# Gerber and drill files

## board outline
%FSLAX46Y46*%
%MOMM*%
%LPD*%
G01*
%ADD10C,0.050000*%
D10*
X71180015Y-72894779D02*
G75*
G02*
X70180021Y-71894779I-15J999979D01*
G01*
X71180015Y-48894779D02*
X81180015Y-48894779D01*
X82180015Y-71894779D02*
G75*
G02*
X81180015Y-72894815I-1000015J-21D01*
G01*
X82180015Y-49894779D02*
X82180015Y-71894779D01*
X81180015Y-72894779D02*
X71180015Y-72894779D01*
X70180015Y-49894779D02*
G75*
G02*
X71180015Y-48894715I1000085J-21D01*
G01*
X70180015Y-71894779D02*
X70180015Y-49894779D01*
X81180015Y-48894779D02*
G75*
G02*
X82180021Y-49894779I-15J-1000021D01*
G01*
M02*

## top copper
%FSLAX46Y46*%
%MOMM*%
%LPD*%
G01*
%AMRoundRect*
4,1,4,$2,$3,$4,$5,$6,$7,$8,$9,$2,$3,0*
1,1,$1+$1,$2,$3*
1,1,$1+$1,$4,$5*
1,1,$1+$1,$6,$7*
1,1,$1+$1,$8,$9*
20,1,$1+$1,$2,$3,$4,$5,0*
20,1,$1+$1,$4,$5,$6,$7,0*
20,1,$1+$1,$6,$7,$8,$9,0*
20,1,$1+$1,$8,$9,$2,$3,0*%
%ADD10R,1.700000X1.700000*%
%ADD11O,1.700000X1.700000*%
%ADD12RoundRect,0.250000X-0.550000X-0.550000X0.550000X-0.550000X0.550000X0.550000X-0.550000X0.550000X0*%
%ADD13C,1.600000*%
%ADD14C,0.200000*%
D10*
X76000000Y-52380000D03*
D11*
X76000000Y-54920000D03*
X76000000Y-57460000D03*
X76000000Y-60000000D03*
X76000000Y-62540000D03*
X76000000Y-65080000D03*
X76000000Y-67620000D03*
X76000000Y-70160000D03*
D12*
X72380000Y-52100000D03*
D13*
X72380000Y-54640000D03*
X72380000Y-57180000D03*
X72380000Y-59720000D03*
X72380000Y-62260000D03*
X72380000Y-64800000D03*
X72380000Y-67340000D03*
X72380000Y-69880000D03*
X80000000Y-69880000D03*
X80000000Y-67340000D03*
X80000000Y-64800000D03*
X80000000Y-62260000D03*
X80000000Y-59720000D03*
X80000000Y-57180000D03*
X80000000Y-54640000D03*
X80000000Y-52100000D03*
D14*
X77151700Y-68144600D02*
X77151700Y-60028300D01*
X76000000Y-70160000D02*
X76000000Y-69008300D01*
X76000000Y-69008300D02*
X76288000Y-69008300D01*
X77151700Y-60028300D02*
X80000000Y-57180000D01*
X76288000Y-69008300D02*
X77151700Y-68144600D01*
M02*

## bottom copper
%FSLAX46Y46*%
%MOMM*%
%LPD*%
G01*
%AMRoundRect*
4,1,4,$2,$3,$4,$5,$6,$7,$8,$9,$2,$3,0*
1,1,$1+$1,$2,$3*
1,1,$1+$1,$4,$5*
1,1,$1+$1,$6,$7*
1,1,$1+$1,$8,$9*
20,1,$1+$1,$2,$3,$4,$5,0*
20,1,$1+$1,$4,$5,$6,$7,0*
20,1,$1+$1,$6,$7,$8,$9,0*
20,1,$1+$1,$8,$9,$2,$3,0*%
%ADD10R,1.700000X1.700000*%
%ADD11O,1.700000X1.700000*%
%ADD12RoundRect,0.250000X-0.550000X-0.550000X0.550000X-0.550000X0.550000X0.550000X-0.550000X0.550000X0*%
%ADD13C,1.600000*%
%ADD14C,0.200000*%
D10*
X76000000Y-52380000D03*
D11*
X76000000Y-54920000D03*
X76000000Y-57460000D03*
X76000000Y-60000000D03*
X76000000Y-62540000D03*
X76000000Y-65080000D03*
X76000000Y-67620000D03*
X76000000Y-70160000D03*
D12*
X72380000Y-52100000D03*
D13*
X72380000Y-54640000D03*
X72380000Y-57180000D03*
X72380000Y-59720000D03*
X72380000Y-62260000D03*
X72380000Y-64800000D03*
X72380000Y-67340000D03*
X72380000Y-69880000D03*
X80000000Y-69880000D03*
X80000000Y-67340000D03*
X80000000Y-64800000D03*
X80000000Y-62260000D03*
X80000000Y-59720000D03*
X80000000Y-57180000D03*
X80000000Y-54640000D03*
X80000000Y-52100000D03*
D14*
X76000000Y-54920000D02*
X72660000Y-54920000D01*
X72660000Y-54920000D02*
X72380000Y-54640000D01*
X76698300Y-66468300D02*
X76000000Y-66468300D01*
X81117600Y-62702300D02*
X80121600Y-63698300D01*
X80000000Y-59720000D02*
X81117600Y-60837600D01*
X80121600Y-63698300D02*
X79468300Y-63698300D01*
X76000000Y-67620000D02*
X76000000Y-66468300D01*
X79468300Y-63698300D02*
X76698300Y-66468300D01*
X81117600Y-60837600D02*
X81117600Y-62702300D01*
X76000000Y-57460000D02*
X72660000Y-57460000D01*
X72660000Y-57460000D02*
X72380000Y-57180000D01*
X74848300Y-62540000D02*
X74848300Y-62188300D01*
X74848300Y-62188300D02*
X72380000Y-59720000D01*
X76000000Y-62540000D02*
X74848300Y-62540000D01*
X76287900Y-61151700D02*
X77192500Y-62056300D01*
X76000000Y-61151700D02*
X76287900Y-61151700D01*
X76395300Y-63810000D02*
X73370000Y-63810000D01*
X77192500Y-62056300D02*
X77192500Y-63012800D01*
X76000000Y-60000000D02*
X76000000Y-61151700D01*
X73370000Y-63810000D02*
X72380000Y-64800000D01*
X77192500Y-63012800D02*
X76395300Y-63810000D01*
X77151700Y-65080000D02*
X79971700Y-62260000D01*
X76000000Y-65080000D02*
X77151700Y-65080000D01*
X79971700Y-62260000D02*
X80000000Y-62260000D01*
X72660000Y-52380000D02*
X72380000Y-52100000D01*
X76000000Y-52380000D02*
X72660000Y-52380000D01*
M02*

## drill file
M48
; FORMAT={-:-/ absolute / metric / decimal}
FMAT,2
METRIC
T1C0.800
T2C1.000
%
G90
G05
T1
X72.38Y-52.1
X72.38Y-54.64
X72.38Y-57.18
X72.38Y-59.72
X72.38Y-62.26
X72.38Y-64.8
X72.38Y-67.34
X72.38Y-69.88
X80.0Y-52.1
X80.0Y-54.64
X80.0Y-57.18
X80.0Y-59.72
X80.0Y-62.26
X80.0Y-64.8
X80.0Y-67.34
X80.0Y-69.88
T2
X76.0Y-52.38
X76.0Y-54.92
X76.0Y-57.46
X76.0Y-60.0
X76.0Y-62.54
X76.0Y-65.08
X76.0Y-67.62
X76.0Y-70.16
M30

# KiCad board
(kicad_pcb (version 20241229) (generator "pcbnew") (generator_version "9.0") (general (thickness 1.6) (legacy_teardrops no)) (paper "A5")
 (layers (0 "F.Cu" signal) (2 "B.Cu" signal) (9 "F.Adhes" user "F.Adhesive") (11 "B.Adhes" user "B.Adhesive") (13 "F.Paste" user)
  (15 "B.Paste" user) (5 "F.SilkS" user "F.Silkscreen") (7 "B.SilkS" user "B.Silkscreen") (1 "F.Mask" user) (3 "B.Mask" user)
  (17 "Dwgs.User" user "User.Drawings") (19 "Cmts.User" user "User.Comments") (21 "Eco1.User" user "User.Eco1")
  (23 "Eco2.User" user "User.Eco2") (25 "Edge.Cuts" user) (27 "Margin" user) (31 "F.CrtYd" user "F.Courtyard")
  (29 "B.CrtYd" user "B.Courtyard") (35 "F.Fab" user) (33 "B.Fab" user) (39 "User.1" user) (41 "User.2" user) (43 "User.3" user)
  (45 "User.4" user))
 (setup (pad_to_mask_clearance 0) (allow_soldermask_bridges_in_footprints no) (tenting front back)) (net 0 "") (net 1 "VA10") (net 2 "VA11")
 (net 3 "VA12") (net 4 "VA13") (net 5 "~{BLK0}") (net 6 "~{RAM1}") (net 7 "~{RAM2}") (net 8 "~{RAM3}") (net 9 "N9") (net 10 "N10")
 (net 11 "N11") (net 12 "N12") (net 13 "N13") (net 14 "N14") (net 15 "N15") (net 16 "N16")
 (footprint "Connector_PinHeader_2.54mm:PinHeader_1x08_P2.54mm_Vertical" (layer "F.Cu") (at 76 52.38)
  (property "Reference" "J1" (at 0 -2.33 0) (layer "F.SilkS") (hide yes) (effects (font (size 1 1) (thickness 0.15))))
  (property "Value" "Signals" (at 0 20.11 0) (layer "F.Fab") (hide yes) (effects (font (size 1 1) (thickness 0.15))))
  (pad "1" thru_hole rect (at 0 0) (size 1.7 1.7) (drill 1) (layers "*.Cu" "*.Mask") (remove_unused_layers no) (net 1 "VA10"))
  (pad "2" thru_hole oval (at 0 2.54) (size 1.7 1.7) (drill 1) (layers "*.Cu" "*.Mask") (remove_unused_layers no) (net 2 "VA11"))
  (pad "3" thru_hole oval (at 0 5.08) (size 1.7 1.7) (drill 1) (layers "*.Cu" "*.Mask") (remove_unused_layers no) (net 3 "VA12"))
  (pad "4" thru_hole oval (at 0 7.62) (size 1.7 1.7) (drill 1) (layers "*.Cu" "*.Mask") (remove_unused_layers no) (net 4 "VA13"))
  (pad "5" thru_hole oval (at 0 10.16) (size 1.7 1.7) (drill 1) (layers "*.Cu" "*.Mask") (remove_unused_layers no) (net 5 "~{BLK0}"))
  (pad "6" thru_hole oval (at 0 12.7) (size 1.7 1.7) (drill 1) (layers "*.Cu" "*.Mask") (remove_unused_layers no) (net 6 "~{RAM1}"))
  (pad "7" thru_hole oval (at 0 15.24) (size 1.7 1.7) (drill 1) (layers "*.Cu" "*.Mask") (remove_unused_layers no) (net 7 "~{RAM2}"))
  (pad "8" thru_hole oval (at 0 17.78) (size 1.7 1.7) (drill 1) (layers "*.Cu" "*.Mask") (remove_unused_layers no) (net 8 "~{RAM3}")))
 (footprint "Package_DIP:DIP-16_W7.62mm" (layer "F.Cu") (at 72.38 52.1)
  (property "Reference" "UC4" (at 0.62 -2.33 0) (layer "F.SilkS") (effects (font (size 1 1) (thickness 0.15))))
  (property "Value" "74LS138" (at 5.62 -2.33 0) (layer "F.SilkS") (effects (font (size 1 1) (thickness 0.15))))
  (pad "1" thru_hole roundrect (at 0 0) (size 1.6 1.6) (drill 0.8) (layers "*.Cu" "*.Mask") (remove_unused_layers no)
   (roundrect_rratio 0.15625) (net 1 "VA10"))
  (pad "2" thru_hole circle (at 0 2.54) (size 1.6 1.6) (drill 0.8) (layers "*.Cu" "*.Mask") (remove_unused_layers no) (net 2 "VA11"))
  (pad "3" thru_hole circle (at 0 5.08) (size 1.6 1.6) (drill 0.8) (layers "*.Cu" "*.Mask") (remove_unused_layers no) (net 3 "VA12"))
  (pad "4" thru_hole circle (at 0 7.62) (size 1.6 1.6) (drill 0.8) (layers "*.Cu" "*.Mask") (remove_unused_layers no) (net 5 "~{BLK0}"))
  (pad "5" thru_hole circle (at 0 10.16) (size 1.6 1.6) (drill 0.8) (layers "*.Cu" "*.Mask") (remove_unused_layers no) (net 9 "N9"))
  (pad "6" thru_hole circle (at 0 12.7) (size 1.6 1.6) (drill 0.8) (layers "*.Cu" "*.Mask") (remove_unused_layers no) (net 4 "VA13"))
  (pad "7" thru_hole circle (at 0 15.24) (size 1.6 1.6) (drill 0.8) (layers "*.Cu" "*.Mask") (remove_unused_layers no) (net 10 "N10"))
  (pad "8" thru_hole circle (at 0 17.78) (size 1.6 1.6) (drill 0.8) (layers "*.Cu" "*.Mask") (remove_unused_layers no) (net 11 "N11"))
  (pad "9" thru_hole circle (at 7.62 17.78) (size 1.6 1.6) (drill 0.8) (layers "*.Cu" "*.Mask") (remove_unused_layers no) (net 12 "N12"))
  (pad "10" thru_hole circle (at 7.62 15.24) (size 1.6 1.6) (drill 0.8) (layers "*.Cu" "*.Mask") (remove_unused_layers no) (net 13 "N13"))
  (pad "11" thru_hole circle (at 7.62 12.7) (size 1.6 1.6) (drill 0.8) (layers "*.Cu" "*.Mask") (remove_unused_layers no) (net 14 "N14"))
  (pad "12" thru_hole circle (at 7.62 10.16) (size 1.6 1.6) (drill 0.8) (layers "*.Cu" "*.Mask") (remove_unused_layers no) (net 6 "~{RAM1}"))
  (pad "13" thru_hole circle (at 7.62 7.62) (size 1.6 1.6) (drill 0.8) (layers "*.Cu" "*.Mask") (remove_unused_layers no) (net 7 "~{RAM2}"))
  (pad "14" thru_hole circle (at 7.62 5.08) (size 1.6 1.6) (drill 0.8) (layers "*.Cu" "*.Mask") (remove_unused_layers no) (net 8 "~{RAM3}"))
  (pad "15" thru_hole circle (at 7.62 2.54) (size 1.6 1.6) (drill 0.8) (layers "*.Cu" "*.Mask") (remove_unused_layers no) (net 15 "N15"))
  (pad "16" thru_hole circle (at 7.62 0) (size 1.6 1.6) (drill 0.8) (layers "*.Cu" "*.Mask") (remove_unused_layers no) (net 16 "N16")))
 (gr_arc (start 71.180015 72.894779) (mid 70.472906 72.60189) (end 70.180015 71.894779) (stroke (width 0.05) (type default))
  (layer "Edge.Cuts"))
 (gr_line (start 71.180015 48.894779) (end 81.180015 48.894779) (stroke (width 0.05) (type default)) (layer "Edge.Cuts"))
 (gr_arc (start 82.180015 71.894779) (mid 81.887122 72.601886) (end 81.180015 72.894779) (stroke (width 0.05) (type default))
  (layer "Edge.Cuts"))
 (gr_line (start 82.180015 49.894779) (end 82.180015 71.894779) (stroke (width 0.05) (type default)) (layer "Edge.Cuts"))
 (gr_line (start 81.180015 72.894779) (end 71.180015 72.894779) (stroke (width 0.05) (type default)) (layer "Edge.Cuts"))
 (gr_arc (start 70.180015 49.894779) (mid 70.472917 49.187691) (end 71.180015 48.894779) (stroke (width 0.05) (type default))
  (layer "Edge.Cuts"))
 (gr_line (start 70.180015 71.894779) (end 70.180015 49.894779) (stroke (width 0.05) (type default)) (layer "Edge.Cuts"))
 (gr_arc (start 81.180015 48.894779) (mid 81.887122 49.187672) (end 82.180015 49.894779) (stroke (width 0.05) (type default))
  (layer "Edge.Cuts"))
 (segment (start 76 54.92) (end 72.66 54.92) (width 0.2) (layer "B.Cu") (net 2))
 (segment (start 72.66 54.92) (end 72.38 54.64) (width 0.2) (layer "B.Cu") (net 2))
 (segment (start 76.6983 66.4683) (end 76 66.4683) (width 0.2) (layer "B.Cu") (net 7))
 (segment (start 81.1176 62.7023) (end 80.1216 63.6983) (width 0.2) (layer "B.Cu") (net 7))
 (segment (start 80 59.72) (end 81.1176 60.8376) (width 0.2) (layer "B.Cu") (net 7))
 (segment (start 80.1216 63.6983) (end 79.4683 63.6983) (width 0.2) (layer "B.Cu") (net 7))
 (segment (start 76 67.62) (end 76 66.4683) (width 0.2) (layer "B.Cu") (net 7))
 (segment (start 79.4683 63.6983) (end 76.6983 66.4683) (width 0.2) (layer "B.Cu") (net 7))
 (segment (start 81.1176 60.8376) (end 81.1176 62.7023) (width 0.2) (layer "B.Cu") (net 7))
 (segment (start 77.1517 68.1446) (end 77.1517 60.0283) (width 0.2) (layer "F.Cu") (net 8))
 (segment (start 76 70.16) (end 76 69.0083) (width 0.2) (layer "F.Cu") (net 8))
 (segment (start 76 69.0083) (end 76.288 69.0083) (width 0.2) (layer "F.Cu") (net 8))
 (segment (start 77.1517 60.0283) (end 80 57.18) (width 0.2) (layer "F.Cu") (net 8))
 (segment (start 76.288 69.0083) (end 77.1517 68.1446) (width 0.2) (layer "F.Cu") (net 8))
 (segment (start 76 57.46) (end 72.66 57.46) (width 0.2) (layer "B.Cu") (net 3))
 (segment (start 72.66 57.46) (end 72.38 57.18) (width 0.2) (layer "B.Cu") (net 3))
 (segment (start 74.8483 62.54) (end 74.8483 62.1883) (width 0.2) (layer "B.Cu") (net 5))
 (segment (start 74.8483 62.1883) (end 72.38 59.72) (width 0.2) (layer "B.Cu") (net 5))
 (segment (start 76 62.54) (end 74.8483 62.54) (width 0.2) (layer "B.Cu") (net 5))
 (segment (start 76.2879 61.1517) (end 77.1925 62.0563) (width 0.2) (layer "B.Cu") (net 4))
 (segment (start 76 61.1517) (end 76.2879 61.1517) (width 0.2) (layer "B.Cu") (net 4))
 (segment (start 76.3953 63.81) (end 73.37 63.81) (width 0.2) (layer "B.Cu") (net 4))
 (segment (start 77.1925 62.0563) (end 77.1925 63.0128) (width 0.2) (layer "B.Cu") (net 4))
 (segment (start 76 60) (end 76 61.1517) (width 0.2) (layer "B.Cu") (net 4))
 (segment (start 73.37 63.81) (end 72.38 64.8) (width 0.2) (layer "B.Cu") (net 4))
 (segment (start 77.1925 63.0128) (end 76.3953 63.81) (width 0.2) (layer "B.Cu") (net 4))
 (segment (start 77.1517 65.08) (end 79.9717 62.26) (width 0.2) (layer "B.Cu") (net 6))
 (segment (start 76 65.08) (end 77.1517 65.08) (width 0.2) (layer "B.Cu") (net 6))
 (segment (start 79.9717 62.26) (end 80 62.26) (width 0.2) (layer "B.Cu") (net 6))
 (segment (start 72.66 52.38) (end 72.38 52.1) (width 0.2) (layer "B.Cu") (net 1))
 (segment (start 76 52.38) (end 72.66 52.38) (width 0.2) (layer "B.Cu") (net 1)))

